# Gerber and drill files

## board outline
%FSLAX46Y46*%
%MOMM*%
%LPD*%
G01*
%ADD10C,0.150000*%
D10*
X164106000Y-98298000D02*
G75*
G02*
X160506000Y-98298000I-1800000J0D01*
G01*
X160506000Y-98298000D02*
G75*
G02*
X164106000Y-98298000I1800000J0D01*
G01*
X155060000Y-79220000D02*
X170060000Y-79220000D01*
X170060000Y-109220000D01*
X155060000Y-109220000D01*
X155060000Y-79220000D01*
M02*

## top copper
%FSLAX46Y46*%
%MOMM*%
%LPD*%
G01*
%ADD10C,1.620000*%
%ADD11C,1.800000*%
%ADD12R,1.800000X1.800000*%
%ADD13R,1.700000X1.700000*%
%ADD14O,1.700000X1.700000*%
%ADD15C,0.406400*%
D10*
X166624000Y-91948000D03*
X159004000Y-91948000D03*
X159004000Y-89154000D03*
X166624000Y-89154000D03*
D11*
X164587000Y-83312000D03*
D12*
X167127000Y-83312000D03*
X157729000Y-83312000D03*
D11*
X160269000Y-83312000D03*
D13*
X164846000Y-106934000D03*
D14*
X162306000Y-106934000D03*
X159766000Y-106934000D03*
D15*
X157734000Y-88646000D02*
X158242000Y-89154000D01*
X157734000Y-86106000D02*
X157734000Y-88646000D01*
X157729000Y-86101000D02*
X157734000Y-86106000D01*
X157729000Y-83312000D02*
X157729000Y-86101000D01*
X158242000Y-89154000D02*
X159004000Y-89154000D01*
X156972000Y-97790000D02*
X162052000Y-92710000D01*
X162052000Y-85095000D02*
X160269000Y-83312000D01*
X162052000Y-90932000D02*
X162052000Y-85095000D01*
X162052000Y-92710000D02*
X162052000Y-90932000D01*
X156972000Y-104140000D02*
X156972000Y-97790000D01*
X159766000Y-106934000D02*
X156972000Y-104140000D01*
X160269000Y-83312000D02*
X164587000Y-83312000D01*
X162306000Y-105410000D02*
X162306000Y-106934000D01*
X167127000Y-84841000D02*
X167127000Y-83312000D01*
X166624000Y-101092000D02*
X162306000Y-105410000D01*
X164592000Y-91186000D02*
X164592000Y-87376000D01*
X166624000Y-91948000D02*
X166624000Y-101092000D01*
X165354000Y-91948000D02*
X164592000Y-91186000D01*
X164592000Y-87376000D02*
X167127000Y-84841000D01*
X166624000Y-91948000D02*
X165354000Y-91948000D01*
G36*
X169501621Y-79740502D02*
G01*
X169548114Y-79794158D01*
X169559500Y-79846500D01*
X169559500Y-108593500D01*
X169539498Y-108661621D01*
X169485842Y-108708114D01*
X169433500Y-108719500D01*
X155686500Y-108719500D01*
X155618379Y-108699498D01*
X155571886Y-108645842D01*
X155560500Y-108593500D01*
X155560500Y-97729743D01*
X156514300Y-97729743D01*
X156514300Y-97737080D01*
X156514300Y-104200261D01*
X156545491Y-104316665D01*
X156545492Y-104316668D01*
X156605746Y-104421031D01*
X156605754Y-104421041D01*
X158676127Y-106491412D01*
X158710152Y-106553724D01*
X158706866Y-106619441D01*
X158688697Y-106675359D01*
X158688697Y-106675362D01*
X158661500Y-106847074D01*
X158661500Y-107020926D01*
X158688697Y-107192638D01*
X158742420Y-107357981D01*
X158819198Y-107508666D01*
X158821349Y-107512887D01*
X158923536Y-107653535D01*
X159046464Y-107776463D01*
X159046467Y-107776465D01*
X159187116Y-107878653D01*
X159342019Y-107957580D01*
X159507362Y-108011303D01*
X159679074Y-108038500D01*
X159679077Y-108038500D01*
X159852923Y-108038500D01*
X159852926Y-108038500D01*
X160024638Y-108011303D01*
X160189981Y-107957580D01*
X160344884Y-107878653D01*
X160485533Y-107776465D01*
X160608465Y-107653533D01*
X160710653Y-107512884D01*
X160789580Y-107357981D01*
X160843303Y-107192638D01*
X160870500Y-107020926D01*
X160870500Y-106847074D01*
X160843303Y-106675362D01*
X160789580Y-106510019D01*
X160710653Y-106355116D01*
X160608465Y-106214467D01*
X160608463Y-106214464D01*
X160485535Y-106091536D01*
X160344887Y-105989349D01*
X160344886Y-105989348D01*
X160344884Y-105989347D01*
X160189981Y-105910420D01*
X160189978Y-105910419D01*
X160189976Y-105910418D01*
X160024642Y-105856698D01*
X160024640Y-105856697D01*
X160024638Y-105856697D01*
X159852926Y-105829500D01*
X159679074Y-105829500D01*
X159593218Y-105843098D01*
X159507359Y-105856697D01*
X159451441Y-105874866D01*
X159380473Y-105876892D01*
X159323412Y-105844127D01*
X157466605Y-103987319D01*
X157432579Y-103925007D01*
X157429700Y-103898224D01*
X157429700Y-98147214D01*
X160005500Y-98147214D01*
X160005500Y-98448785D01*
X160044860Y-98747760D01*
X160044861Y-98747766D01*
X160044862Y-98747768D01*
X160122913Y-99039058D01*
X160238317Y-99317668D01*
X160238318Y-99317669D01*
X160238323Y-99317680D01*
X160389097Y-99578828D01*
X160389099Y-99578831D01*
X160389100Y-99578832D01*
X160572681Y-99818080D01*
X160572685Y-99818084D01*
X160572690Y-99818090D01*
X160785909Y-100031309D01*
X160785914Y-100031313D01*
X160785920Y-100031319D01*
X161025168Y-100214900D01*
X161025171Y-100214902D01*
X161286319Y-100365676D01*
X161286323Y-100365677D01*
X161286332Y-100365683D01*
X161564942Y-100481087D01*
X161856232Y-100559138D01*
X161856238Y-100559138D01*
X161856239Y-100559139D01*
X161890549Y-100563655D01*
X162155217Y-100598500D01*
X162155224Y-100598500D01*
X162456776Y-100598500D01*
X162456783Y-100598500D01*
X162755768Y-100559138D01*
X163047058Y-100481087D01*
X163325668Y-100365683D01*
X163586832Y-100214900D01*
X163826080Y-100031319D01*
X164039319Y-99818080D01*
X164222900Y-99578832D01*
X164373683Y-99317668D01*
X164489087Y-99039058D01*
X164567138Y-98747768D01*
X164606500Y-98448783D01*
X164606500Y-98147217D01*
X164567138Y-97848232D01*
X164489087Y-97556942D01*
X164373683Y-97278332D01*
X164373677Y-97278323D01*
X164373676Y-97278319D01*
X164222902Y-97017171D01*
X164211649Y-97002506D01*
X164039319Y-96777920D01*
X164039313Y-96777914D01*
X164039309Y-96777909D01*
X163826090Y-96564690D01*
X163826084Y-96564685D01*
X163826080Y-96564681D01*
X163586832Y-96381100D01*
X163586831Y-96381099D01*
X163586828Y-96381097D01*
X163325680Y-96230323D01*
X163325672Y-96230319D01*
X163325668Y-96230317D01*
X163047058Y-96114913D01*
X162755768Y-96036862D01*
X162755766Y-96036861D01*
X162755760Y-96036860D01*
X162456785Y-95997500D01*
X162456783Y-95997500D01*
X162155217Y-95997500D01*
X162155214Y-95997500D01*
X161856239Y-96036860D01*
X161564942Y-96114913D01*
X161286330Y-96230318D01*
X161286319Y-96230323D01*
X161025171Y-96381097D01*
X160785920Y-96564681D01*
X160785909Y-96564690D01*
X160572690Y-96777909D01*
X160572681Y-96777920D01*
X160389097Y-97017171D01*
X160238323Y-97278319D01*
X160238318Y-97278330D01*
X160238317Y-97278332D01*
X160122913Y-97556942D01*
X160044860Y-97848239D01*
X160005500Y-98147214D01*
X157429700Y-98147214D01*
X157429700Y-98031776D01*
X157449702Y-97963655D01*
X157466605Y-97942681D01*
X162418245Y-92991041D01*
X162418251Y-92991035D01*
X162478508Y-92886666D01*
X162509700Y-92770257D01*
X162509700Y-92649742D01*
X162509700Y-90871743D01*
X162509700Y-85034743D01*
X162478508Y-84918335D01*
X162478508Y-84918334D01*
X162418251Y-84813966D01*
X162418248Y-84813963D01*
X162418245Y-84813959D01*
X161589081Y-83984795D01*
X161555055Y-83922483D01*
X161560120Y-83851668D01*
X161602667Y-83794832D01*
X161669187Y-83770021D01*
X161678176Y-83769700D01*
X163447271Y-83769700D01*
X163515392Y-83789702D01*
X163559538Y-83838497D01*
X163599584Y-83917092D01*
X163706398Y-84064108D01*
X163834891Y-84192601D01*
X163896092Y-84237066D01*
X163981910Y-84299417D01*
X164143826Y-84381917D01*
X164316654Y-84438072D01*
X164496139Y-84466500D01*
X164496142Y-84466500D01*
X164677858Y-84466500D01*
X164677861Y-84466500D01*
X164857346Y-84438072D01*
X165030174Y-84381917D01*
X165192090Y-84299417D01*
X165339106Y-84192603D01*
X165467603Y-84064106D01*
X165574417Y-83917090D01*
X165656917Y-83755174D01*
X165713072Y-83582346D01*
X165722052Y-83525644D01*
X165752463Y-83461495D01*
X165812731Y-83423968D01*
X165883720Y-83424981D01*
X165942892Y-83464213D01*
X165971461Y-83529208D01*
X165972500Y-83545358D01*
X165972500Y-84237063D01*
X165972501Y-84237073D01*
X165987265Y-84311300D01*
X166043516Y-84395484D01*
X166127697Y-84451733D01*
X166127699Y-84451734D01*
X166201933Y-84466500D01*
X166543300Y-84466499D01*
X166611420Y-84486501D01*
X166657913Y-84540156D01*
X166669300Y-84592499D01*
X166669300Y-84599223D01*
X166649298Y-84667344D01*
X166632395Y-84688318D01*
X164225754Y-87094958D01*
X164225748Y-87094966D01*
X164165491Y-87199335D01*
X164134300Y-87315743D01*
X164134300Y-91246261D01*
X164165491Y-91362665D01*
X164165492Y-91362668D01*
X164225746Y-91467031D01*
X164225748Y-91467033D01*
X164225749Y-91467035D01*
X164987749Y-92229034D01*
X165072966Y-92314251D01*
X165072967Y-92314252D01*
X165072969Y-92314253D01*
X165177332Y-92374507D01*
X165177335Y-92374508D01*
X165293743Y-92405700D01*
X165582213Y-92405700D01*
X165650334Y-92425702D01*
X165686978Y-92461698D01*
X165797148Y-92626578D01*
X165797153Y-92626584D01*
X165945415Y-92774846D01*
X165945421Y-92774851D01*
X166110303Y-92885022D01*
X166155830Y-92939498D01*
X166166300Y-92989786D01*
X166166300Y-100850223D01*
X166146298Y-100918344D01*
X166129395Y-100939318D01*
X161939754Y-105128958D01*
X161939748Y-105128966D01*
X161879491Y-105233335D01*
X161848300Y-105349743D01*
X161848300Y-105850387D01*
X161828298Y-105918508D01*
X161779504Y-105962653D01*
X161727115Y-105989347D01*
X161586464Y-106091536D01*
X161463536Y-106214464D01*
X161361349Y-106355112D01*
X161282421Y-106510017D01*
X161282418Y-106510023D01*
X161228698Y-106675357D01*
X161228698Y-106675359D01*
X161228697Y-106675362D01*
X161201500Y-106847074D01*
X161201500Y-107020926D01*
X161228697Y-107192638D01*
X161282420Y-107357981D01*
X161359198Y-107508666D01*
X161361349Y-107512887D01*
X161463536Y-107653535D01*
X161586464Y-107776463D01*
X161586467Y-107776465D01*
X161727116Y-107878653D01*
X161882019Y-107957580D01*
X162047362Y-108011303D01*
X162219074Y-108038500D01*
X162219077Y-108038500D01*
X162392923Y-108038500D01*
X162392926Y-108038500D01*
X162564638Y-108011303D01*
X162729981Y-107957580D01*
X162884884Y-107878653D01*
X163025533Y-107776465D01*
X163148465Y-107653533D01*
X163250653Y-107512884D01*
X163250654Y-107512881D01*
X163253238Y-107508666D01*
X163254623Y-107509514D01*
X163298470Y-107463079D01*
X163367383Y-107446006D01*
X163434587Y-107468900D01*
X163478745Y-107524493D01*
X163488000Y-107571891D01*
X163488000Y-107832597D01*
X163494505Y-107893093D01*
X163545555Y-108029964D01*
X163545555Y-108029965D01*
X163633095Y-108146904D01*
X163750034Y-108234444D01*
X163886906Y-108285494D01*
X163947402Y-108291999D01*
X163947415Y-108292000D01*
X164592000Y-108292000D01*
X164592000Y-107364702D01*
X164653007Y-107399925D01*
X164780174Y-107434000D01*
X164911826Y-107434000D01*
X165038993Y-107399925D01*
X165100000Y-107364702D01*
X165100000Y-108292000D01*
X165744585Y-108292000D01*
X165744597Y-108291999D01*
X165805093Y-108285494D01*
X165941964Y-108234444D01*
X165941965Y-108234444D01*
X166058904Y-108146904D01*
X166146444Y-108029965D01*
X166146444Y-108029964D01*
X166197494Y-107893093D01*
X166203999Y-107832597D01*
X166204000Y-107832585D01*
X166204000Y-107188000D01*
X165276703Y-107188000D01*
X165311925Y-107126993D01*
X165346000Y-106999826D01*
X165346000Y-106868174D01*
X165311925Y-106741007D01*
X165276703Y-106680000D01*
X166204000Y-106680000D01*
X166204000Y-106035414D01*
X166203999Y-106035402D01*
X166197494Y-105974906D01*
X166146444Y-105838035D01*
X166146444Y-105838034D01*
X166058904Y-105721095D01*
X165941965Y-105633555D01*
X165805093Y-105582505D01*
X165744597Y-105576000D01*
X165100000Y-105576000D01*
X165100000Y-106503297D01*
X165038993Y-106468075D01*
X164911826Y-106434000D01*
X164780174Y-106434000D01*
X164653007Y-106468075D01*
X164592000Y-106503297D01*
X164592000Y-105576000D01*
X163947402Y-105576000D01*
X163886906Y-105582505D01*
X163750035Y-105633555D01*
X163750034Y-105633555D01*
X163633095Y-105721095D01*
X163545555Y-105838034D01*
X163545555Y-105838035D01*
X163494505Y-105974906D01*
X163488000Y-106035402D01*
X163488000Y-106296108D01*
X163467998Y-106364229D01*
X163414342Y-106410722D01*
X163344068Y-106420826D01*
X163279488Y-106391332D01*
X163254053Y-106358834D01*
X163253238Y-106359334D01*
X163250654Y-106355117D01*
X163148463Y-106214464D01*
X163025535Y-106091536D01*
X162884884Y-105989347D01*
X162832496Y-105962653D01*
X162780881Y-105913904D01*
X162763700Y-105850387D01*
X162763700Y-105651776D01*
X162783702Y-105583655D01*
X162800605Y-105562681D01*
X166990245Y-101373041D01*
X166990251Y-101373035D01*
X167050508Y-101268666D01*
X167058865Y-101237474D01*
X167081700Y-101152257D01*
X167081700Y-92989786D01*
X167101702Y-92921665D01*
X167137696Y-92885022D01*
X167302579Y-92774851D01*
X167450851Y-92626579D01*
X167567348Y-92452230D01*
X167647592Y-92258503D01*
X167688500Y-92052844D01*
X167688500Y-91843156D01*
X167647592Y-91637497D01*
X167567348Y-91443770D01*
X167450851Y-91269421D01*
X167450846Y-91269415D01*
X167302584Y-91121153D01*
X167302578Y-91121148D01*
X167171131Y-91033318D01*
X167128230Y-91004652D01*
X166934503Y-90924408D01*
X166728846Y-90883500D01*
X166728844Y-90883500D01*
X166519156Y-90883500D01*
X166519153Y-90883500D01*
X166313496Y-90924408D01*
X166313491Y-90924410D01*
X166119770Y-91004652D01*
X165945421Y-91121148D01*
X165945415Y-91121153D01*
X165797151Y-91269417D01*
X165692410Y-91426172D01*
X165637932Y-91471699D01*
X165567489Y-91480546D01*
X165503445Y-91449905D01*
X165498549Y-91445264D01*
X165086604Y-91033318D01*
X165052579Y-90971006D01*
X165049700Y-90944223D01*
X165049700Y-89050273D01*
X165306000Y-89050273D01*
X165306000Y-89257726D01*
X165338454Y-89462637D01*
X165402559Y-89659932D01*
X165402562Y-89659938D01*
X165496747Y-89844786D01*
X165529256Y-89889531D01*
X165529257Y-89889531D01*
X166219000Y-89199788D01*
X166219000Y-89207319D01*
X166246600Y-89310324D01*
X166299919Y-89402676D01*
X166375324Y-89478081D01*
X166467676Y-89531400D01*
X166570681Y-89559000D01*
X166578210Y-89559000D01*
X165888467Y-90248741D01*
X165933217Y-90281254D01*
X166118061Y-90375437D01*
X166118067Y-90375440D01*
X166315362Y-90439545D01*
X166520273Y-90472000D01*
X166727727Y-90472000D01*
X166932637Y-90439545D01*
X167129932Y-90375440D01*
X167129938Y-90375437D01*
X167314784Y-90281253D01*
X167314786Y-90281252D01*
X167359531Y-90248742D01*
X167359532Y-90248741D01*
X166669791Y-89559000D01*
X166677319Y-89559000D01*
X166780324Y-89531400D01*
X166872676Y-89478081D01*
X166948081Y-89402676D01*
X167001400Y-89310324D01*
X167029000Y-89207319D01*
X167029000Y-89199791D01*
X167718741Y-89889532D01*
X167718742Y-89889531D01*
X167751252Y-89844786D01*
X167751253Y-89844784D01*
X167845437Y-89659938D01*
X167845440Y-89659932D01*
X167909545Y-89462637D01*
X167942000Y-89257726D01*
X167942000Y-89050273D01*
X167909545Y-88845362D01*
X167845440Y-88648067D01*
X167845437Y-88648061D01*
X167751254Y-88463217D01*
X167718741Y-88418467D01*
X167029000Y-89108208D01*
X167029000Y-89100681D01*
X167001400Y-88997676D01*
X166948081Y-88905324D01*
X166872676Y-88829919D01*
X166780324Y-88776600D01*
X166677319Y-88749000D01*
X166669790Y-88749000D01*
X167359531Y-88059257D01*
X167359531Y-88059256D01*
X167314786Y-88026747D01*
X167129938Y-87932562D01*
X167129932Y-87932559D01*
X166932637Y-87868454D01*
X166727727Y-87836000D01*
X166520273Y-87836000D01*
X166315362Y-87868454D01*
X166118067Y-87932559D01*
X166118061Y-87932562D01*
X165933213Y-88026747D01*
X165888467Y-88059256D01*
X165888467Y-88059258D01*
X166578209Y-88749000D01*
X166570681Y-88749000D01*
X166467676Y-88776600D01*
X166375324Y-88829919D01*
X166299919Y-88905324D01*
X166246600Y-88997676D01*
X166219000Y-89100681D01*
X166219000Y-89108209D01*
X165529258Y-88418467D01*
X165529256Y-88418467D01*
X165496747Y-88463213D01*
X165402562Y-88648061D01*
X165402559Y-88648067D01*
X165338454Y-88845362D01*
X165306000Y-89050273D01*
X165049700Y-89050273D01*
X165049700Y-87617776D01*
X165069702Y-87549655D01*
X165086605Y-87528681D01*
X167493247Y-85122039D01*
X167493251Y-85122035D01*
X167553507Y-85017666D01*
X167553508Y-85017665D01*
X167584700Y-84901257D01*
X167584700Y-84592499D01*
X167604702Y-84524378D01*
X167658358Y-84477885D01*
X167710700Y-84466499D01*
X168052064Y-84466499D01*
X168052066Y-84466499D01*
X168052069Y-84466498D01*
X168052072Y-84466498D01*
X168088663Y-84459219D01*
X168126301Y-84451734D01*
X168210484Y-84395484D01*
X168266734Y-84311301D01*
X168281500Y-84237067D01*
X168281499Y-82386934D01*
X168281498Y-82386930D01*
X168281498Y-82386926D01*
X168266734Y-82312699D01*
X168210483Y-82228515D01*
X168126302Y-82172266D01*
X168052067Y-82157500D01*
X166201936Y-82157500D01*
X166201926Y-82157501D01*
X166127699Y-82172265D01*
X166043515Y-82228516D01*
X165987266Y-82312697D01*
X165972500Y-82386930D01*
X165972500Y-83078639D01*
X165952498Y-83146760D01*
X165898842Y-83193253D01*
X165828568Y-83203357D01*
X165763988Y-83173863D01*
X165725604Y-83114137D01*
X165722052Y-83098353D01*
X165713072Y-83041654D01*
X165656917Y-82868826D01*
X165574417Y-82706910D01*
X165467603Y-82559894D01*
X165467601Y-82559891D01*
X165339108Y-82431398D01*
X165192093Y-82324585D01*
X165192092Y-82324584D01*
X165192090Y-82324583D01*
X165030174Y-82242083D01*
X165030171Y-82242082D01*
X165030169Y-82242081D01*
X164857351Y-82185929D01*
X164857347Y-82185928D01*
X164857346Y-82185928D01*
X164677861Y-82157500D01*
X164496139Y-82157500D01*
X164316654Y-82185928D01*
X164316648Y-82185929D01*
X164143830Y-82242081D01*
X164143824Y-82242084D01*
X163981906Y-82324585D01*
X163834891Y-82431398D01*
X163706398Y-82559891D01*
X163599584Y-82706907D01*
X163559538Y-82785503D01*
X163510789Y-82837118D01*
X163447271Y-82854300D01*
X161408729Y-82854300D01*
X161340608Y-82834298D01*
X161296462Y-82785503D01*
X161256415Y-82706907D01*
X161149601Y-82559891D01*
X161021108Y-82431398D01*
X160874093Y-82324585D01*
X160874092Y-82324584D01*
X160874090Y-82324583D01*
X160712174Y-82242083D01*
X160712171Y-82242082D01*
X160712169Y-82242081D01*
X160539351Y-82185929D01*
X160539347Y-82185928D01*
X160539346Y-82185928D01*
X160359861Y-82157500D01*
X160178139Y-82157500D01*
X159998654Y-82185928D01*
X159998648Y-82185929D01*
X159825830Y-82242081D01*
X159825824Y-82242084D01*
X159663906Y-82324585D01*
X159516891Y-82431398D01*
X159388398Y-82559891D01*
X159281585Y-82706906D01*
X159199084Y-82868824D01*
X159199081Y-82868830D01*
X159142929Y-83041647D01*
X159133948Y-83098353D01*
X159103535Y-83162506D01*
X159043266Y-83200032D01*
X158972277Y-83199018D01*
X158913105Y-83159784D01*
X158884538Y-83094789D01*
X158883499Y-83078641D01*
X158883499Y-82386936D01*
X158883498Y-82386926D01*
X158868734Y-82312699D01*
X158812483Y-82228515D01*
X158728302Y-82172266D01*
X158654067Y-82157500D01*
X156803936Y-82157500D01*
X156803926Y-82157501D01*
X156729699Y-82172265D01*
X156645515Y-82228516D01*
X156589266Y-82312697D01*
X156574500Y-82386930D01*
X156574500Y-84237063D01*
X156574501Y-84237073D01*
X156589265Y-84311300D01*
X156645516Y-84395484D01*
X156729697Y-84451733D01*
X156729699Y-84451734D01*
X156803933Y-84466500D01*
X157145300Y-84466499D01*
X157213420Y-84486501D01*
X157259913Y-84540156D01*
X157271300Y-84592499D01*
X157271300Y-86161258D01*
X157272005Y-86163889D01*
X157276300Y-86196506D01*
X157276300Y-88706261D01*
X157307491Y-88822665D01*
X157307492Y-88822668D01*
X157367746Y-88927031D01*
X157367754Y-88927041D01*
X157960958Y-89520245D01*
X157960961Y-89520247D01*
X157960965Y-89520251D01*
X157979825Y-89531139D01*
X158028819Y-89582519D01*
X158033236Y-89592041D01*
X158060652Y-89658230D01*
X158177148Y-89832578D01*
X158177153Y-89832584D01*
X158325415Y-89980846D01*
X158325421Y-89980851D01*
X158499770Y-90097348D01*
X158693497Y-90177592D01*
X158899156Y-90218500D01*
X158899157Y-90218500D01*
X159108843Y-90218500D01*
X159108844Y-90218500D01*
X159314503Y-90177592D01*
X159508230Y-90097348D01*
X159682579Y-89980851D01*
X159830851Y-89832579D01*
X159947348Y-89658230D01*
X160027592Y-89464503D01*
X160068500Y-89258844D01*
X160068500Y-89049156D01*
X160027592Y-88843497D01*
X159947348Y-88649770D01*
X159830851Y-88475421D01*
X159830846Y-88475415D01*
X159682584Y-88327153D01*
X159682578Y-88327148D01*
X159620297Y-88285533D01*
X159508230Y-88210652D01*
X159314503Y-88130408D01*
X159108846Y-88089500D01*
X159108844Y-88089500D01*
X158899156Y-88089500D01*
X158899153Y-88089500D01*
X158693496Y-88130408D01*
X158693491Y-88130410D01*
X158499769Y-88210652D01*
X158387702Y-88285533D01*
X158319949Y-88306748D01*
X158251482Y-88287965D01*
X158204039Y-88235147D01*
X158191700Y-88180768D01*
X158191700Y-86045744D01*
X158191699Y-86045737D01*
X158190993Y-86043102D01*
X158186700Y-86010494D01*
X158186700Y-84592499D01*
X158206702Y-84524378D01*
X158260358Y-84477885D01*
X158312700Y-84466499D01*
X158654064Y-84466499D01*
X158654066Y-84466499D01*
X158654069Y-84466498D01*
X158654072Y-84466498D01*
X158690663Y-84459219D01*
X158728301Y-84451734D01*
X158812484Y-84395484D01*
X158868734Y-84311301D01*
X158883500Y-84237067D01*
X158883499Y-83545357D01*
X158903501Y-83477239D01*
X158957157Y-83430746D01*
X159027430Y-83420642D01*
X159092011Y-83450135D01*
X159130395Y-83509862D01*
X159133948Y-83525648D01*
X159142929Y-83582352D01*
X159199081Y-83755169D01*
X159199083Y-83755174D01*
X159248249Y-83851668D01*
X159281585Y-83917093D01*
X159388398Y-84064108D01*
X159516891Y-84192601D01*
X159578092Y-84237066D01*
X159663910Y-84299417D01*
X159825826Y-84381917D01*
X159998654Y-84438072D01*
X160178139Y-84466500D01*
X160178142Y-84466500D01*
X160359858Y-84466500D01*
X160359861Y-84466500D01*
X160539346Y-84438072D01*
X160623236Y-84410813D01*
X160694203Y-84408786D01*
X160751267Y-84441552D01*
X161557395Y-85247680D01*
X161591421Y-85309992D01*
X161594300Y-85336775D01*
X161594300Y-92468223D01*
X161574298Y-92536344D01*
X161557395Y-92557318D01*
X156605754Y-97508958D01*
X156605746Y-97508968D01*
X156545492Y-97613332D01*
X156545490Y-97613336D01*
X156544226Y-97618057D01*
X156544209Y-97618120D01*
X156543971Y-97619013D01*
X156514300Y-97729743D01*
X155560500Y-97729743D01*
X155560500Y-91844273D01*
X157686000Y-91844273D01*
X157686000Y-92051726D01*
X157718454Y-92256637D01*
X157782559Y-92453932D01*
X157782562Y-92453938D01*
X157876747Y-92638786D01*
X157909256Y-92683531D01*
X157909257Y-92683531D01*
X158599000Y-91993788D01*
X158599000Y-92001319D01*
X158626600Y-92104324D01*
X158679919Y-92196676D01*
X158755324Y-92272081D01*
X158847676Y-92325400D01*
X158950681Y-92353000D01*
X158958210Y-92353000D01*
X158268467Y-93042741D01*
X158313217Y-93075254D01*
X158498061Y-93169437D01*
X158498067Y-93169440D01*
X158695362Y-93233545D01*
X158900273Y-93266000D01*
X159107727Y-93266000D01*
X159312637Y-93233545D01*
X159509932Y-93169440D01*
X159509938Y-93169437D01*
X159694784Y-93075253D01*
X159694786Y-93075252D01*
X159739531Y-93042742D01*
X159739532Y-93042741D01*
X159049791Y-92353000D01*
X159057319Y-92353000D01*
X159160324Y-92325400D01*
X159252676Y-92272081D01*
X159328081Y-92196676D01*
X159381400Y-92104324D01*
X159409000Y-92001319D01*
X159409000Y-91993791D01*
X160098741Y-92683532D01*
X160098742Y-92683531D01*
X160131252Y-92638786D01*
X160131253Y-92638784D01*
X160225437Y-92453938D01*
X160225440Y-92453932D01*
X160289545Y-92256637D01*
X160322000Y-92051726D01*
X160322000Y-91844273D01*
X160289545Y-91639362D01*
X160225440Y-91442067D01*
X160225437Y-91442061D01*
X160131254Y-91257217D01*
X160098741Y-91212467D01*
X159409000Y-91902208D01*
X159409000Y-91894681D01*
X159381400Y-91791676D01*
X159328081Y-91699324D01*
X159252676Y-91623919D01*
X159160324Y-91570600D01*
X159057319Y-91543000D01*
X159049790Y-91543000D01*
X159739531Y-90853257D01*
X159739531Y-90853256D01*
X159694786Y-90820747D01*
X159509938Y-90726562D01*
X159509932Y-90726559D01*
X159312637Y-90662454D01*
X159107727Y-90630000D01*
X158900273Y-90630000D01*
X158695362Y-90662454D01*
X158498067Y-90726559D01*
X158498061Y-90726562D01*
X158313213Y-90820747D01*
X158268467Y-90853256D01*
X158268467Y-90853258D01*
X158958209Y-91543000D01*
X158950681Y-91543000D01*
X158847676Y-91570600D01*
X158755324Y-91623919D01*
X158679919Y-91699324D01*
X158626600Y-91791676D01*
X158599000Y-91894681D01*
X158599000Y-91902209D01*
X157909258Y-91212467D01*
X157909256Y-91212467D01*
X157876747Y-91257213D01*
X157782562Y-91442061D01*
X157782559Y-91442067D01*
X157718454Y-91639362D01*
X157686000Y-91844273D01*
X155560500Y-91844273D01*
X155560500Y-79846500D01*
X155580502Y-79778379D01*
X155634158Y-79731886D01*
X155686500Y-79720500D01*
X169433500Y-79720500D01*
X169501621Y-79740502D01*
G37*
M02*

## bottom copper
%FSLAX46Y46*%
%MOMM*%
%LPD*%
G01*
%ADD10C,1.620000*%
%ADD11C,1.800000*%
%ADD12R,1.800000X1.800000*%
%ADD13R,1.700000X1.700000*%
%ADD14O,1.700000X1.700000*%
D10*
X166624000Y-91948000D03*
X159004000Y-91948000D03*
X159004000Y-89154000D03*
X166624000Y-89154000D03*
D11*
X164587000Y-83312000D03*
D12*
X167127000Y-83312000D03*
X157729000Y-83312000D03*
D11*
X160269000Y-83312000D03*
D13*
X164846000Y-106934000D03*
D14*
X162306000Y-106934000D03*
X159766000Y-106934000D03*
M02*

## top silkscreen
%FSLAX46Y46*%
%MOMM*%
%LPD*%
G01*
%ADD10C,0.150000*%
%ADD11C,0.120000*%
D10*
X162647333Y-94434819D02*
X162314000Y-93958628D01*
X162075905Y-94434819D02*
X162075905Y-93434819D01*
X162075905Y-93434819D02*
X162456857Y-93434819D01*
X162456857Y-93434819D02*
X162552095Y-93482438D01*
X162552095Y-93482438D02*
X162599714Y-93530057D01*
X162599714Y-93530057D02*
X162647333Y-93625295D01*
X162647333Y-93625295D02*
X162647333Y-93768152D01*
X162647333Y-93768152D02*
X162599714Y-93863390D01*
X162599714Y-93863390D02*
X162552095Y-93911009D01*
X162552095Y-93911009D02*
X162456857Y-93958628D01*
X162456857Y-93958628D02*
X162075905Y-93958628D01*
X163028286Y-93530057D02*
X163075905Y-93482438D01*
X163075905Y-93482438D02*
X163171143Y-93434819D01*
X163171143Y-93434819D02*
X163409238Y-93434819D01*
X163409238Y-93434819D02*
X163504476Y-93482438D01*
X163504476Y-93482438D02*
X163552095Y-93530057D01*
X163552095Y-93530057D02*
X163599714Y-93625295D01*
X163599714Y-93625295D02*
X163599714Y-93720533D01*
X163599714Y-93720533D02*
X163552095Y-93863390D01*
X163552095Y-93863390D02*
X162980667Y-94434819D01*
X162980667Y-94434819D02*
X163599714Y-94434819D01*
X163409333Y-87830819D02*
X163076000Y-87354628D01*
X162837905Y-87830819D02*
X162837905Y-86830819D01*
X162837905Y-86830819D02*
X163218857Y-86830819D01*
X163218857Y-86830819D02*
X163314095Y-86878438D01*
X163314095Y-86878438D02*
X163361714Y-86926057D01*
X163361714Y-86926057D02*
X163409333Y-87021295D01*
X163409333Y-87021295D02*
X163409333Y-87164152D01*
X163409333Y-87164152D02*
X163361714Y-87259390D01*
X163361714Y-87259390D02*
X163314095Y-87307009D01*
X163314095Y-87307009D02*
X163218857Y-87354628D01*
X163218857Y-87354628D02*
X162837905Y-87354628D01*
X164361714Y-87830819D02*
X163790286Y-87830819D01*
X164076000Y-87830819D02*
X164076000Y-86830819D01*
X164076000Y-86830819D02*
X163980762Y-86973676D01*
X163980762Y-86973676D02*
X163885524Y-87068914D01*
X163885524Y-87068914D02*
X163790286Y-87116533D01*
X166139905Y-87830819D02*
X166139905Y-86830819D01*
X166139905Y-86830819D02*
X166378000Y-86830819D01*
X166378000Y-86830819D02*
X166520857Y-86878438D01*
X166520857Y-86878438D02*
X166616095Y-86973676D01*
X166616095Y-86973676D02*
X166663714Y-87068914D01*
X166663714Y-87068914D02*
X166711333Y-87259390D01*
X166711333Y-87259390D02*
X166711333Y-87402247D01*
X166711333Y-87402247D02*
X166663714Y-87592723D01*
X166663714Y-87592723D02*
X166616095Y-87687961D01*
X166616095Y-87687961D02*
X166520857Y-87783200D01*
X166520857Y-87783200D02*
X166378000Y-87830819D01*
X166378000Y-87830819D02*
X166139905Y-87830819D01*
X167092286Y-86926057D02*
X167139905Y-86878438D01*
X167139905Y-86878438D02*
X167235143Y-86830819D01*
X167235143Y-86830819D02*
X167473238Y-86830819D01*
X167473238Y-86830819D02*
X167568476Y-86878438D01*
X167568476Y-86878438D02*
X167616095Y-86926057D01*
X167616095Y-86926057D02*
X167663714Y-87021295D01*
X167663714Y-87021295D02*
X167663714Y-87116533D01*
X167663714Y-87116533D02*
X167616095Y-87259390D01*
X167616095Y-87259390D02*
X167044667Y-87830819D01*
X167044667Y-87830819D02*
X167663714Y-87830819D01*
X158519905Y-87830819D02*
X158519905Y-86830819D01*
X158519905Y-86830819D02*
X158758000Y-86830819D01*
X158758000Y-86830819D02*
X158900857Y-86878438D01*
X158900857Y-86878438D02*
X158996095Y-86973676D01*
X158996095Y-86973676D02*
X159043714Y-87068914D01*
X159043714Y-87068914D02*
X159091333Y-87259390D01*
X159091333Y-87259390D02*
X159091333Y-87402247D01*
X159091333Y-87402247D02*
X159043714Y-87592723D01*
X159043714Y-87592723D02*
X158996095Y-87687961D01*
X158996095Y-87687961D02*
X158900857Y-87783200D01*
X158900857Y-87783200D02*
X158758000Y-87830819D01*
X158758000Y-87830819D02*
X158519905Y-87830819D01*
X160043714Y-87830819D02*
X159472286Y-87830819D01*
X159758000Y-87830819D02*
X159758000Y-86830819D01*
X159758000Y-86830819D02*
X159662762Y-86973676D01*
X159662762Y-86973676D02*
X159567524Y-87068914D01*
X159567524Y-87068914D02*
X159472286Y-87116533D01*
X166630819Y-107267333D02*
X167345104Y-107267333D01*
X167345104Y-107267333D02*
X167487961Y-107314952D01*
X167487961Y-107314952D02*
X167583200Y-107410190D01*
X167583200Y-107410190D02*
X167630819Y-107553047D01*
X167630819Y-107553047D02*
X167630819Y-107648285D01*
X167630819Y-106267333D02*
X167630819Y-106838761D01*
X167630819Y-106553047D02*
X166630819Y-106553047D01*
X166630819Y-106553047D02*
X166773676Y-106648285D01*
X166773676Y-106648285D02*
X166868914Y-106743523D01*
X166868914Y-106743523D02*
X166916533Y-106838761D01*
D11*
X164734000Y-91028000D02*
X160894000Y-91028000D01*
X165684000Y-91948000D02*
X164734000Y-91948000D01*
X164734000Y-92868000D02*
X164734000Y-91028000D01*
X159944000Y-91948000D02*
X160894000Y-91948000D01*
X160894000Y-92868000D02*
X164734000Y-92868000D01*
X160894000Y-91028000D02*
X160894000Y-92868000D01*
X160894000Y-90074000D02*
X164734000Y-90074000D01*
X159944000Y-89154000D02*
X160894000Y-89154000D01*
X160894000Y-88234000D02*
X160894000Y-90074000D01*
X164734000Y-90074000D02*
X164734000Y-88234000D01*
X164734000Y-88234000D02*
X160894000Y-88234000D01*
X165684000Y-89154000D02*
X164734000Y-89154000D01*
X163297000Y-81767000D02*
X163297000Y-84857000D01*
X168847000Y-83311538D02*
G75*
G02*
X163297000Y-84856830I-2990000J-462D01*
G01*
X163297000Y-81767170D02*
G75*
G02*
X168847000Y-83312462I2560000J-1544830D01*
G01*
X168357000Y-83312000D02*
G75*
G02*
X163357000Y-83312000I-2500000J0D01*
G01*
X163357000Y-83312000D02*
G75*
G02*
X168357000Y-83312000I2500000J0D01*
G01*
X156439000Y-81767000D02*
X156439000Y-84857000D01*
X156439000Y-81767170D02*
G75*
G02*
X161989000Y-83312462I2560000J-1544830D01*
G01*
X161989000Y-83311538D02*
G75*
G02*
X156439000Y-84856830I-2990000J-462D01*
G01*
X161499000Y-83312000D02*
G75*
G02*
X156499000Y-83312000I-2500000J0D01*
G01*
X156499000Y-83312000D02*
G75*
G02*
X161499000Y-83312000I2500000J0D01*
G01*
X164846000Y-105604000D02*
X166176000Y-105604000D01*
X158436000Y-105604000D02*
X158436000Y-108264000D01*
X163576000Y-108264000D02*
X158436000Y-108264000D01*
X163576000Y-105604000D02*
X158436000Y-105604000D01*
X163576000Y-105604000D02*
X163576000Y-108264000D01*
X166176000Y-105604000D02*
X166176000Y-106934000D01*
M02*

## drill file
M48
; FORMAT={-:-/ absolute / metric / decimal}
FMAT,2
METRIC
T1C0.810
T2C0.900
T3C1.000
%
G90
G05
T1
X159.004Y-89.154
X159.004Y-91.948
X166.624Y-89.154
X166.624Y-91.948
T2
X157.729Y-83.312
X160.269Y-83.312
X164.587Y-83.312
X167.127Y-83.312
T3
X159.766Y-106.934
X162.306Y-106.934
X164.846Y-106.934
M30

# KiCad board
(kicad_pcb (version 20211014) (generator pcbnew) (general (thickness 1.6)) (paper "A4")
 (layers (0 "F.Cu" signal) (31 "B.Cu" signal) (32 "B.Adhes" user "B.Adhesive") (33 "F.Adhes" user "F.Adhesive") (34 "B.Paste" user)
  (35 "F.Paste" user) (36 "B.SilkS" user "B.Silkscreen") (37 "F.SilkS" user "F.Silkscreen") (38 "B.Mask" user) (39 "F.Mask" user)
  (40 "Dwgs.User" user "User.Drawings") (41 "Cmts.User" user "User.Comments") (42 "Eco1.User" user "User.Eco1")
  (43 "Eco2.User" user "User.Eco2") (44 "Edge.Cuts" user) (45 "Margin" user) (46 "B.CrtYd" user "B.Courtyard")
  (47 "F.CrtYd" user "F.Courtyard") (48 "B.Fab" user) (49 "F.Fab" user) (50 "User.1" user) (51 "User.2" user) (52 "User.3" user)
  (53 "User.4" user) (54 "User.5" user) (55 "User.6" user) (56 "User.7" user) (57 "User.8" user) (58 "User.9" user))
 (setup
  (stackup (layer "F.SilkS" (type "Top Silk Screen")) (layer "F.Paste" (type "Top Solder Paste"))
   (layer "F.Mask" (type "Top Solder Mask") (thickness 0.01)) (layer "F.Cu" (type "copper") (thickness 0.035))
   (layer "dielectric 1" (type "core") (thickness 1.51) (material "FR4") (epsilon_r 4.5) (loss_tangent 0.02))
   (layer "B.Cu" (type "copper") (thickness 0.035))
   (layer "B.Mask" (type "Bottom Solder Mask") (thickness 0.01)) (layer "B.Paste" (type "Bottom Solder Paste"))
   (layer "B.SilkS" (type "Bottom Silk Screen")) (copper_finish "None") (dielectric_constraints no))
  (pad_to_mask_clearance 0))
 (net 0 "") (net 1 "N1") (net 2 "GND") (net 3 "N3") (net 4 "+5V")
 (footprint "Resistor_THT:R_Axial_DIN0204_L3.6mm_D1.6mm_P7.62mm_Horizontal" (layer "F.Cu") (at 166.624 91.948 180)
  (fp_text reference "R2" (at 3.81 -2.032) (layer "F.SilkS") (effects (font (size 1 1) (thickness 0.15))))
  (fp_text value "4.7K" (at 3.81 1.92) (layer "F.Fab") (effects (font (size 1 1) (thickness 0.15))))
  (fp_line (start 1.89 0.92) (end 5.73 0.92) (layer "F.SilkS") (width 0.12))
  (fp_line (start 0.94 0) (end 1.89 0) (layer "F.SilkS") (width 0.12))
  (fp_line (start 1.89 -0.92) (end 1.89 0.92) (layer "F.SilkS") (width 0.12))
  (fp_line (start 6.68 0) (end 5.73 0) (layer "F.SilkS") (width 0.12))
  (fp_line (start 5.73 -0.92) (end 1.89 -0.92) (layer "F.SilkS") (width 0.12))
  (fp_line (start 5.73 0.92) (end 5.73 -0.92) (layer "F.SilkS") (width 0.12))
  (pad "1" thru_hole circle (at 0 0 180) (size 1.62 1.62) (drill 0.81) (layers *.Cu *.Mask) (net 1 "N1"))
  (pad "2" thru_hole circle (at 7.62 0 180) (size 1.62 1.62) (drill 0.81) (layers *.Cu *.Mask) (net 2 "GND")))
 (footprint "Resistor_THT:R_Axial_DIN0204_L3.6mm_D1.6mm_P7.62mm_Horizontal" (layer "F.Cu") (at 159.004 89.154)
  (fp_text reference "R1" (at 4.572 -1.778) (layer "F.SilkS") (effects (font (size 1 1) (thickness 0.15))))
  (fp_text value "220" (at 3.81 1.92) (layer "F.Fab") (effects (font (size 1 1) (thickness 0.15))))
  (fp_line (start 1.89 0.92) (end 5.73 0.92) (layer "F.SilkS") (width 0.12))
  (fp_line (start 0.94 0) (end 1.89 0) (layer "F.SilkS") (width 0.12))
  (fp_line (start 1.89 -0.92) (end 1.89 0.92) (layer "F.SilkS") (width 0.12))
  (fp_line (start 5.73 0.92) (end 5.73 -0.92) (layer "F.SilkS") (width 0.12))
  (fp_line (start 5.73 -0.92) (end 1.89 -0.92) (layer "F.SilkS") (width 0.12))
  (fp_line (start 6.68 0) (end 5.73 0) (layer "F.SilkS") (width 0.12))
  (pad "1" thru_hole circle (at 0 0) (size 1.62 1.62) (drill 0.81) (layers *.Cu *.Mask) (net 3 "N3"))
  (pad "2" thru_hole circle (at 7.62 0) (size 1.62 1.62) (drill 0.81) (layers *.Cu *.Mask) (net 2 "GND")))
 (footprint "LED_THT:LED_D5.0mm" (layer "F.Cu") (at 164.587 83.312)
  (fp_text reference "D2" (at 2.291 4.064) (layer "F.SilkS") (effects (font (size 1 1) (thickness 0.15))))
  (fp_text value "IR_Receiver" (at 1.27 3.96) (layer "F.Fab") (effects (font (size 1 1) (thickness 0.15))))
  (fp_line (start -1.29 -1.545) (end -1.29 1.545) (layer "F.SilkS") (width 0.12))
  (fp_arc (start 4.26 -0.000462) (mid 2.072002 2.880433) (end -1.29 1.54483) (layer "F.SilkS") (width 0.12))
  (fp_arc (start -1.29 -1.54483) (mid 2.072002 -2.880433) (end 4.26 0.000462) (layer "F.SilkS") (width 0.12))
  (fp_circle (center 1.27 0) (end 3.77 0) (layer "F.SilkS") (width 0.12) (fill none))
  (pad "1" thru_hole circle (at 0 0) (size 1.8 1.8) (drill 0.9) (layers *.Cu *.Mask) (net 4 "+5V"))
  (pad "2" thru_hole rect (at 2.54 0) (size 1.8 1.8) (drill 0.9) (layers *.Cu *.Mask) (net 1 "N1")))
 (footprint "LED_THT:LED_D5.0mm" (layer "F.Cu") (at 157.729 83.312)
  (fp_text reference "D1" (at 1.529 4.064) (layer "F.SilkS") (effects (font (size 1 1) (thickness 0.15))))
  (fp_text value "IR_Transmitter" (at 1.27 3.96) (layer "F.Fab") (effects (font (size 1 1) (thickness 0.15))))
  (fp_line (start -1.29 -1.545) (end -1.29 1.545) (layer "F.SilkS") (width 0.12))
  (fp_arc (start -1.29 -1.54483) (mid 2.072002 -2.880433) (end 4.26 0.000462) (layer "F.SilkS") (width 0.12))
  (fp_arc (start 4.26 -0.000462) (mid 2.072002 2.880433) (end -1.29 1.54483) (layer "F.SilkS") (width 0.12))
  (fp_circle (center 1.27 0) (end 3.77 0) (layer "F.SilkS") (width 0.12) (fill none))
  (pad "1" thru_hole rect (at 0 0) (size 1.8 1.8) (drill 0.9) (layers *.Cu *.Mask) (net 3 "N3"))
  (pad "2" thru_hole circle (at 2.54 0) (size 1.8 1.8) (drill 0.9) (layers *.Cu *.Mask) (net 4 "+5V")))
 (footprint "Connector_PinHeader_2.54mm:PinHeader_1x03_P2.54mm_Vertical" (layer "F.Cu") (at 164.846 106.934 -90)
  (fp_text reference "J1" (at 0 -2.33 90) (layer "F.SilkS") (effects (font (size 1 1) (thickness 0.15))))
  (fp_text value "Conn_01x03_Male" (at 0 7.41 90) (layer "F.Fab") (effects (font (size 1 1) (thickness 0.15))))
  (fp_line (start -1.33 0) (end -1.33 -1.33) (layer "F.SilkS") (width 0.12))
  (fp_line (start -1.33 6.41) (end 1.33 6.41) (layer "F.SilkS") (width 0.12))
  (fp_line (start 1.33 1.27) (end 1.33 6.41) (layer "F.SilkS") (width 0.12))
  (fp_line (start -1.33 1.27) (end -1.33 6.41) (layer "F.SilkS") (width 0.12))
  (fp_line (start -1.33 1.27) (end 1.33 1.27) (layer "F.SilkS") (width 0.12))
  (fp_line (start -1.33 -1.33) (end 0 -1.33) (layer "F.SilkS") (width 0.12))
  (pad "1" thru_hole rect (at 0 0 270) (size 1.7 1.7) (drill 1) (layers *.Cu *.Mask) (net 2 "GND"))
  (pad "2" thru_hole oval (at 0 2.54 270) (size 1.7 1.7) (drill 1) (layers *.Cu *.Mask) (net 1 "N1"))
  (pad "3" thru_hole oval (at 0 5.08 270) (size 1.7 1.7) (drill 1) (layers *.Cu *.Mask) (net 4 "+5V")))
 (gr_circle (center 162.306 98.298) (end 164.106 98.298) (layer "Edge.Cuts") (width 0.15) (fill none))
 (gr_rect (start 155.06 79.22) (end 170.06 109.22) (layer "Edge.Cuts") (width 0.15) (fill none))
 (segment (start 157.734 88.646) (end 158.242 89.154) (width 0.4064) (layer "F.Cu") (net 3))
 (segment (start 157.734 86.106) (end 157.734 88.646) (width 0.4064) (layer "F.Cu") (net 3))
 (segment (start 157.729 86.101) (end 157.734 86.106) (width 0.4064) (layer "F.Cu") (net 3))
 (segment (start 157.729 83.312) (end 157.729 86.101) (width 0.4064) (layer "F.Cu") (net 3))
 (segment (start 158.242 89.154) (end 159.004 89.154) (width 0.4064) (layer "F.Cu") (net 3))
 (segment (start 156.972 97.79) (end 162.052 92.71) (width 0.4064) (layer "F.Cu") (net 4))
 (segment (start 162.052 85.095) (end 160.269 83.312) (width 0.4064) (layer "F.Cu") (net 4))
 (segment (start 162.052 90.932) (end 162.052 85.095) (width 0.4064) (layer "F.Cu") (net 4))
 (segment (start 162.052 92.71) (end 162.052 90.932) (width 0.4064) (layer "F.Cu") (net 4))
 (segment (start 156.972 104.14) (end 156.972 97.79) (width 0.4064) (layer "F.Cu") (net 4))
 (segment (start 159.766 106.934) (end 156.972 104.14) (width 0.4064) (layer "F.Cu") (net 4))
 (segment (start 160.269 83.312) (end 164.587 83.312) (width 0.4064) (layer "F.Cu") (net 4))
 (segment (start 162.306 105.41) (end 162.306 106.934) (width 0.4064) (layer "F.Cu") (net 1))
 (segment (start 167.127 84.841) (end 167.127 83.312) (width 0.4064) (layer "F.Cu") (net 1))
 (segment (start 166.624 101.092) (end 162.306 105.41) (width 0.4064) (layer "F.Cu") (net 1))
 (segment (start 164.592 91.186) (end 164.592 87.376) (width 0.4064) (layer "F.Cu") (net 1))
 (segment (start 166.624 91.948) (end 166.624 101.092) (width 0.4064) (layer "F.Cu") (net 1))
 (segment (start 165.354 91.948) (end 164.592 91.186) (width 0.4064) (layer "F.Cu") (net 1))
 (segment (start 164.592 87.376) (end 167.127 84.841) (width 0.4064) (layer "F.Cu") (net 1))
 (segment (start 166.624 91.948) (end 165.354 91.948) (width 0.4064) (layer "F.Cu") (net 1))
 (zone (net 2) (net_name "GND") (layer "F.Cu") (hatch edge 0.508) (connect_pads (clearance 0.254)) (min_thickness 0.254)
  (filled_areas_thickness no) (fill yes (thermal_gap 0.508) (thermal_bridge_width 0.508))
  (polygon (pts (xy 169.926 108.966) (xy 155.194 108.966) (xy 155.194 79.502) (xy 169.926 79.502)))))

